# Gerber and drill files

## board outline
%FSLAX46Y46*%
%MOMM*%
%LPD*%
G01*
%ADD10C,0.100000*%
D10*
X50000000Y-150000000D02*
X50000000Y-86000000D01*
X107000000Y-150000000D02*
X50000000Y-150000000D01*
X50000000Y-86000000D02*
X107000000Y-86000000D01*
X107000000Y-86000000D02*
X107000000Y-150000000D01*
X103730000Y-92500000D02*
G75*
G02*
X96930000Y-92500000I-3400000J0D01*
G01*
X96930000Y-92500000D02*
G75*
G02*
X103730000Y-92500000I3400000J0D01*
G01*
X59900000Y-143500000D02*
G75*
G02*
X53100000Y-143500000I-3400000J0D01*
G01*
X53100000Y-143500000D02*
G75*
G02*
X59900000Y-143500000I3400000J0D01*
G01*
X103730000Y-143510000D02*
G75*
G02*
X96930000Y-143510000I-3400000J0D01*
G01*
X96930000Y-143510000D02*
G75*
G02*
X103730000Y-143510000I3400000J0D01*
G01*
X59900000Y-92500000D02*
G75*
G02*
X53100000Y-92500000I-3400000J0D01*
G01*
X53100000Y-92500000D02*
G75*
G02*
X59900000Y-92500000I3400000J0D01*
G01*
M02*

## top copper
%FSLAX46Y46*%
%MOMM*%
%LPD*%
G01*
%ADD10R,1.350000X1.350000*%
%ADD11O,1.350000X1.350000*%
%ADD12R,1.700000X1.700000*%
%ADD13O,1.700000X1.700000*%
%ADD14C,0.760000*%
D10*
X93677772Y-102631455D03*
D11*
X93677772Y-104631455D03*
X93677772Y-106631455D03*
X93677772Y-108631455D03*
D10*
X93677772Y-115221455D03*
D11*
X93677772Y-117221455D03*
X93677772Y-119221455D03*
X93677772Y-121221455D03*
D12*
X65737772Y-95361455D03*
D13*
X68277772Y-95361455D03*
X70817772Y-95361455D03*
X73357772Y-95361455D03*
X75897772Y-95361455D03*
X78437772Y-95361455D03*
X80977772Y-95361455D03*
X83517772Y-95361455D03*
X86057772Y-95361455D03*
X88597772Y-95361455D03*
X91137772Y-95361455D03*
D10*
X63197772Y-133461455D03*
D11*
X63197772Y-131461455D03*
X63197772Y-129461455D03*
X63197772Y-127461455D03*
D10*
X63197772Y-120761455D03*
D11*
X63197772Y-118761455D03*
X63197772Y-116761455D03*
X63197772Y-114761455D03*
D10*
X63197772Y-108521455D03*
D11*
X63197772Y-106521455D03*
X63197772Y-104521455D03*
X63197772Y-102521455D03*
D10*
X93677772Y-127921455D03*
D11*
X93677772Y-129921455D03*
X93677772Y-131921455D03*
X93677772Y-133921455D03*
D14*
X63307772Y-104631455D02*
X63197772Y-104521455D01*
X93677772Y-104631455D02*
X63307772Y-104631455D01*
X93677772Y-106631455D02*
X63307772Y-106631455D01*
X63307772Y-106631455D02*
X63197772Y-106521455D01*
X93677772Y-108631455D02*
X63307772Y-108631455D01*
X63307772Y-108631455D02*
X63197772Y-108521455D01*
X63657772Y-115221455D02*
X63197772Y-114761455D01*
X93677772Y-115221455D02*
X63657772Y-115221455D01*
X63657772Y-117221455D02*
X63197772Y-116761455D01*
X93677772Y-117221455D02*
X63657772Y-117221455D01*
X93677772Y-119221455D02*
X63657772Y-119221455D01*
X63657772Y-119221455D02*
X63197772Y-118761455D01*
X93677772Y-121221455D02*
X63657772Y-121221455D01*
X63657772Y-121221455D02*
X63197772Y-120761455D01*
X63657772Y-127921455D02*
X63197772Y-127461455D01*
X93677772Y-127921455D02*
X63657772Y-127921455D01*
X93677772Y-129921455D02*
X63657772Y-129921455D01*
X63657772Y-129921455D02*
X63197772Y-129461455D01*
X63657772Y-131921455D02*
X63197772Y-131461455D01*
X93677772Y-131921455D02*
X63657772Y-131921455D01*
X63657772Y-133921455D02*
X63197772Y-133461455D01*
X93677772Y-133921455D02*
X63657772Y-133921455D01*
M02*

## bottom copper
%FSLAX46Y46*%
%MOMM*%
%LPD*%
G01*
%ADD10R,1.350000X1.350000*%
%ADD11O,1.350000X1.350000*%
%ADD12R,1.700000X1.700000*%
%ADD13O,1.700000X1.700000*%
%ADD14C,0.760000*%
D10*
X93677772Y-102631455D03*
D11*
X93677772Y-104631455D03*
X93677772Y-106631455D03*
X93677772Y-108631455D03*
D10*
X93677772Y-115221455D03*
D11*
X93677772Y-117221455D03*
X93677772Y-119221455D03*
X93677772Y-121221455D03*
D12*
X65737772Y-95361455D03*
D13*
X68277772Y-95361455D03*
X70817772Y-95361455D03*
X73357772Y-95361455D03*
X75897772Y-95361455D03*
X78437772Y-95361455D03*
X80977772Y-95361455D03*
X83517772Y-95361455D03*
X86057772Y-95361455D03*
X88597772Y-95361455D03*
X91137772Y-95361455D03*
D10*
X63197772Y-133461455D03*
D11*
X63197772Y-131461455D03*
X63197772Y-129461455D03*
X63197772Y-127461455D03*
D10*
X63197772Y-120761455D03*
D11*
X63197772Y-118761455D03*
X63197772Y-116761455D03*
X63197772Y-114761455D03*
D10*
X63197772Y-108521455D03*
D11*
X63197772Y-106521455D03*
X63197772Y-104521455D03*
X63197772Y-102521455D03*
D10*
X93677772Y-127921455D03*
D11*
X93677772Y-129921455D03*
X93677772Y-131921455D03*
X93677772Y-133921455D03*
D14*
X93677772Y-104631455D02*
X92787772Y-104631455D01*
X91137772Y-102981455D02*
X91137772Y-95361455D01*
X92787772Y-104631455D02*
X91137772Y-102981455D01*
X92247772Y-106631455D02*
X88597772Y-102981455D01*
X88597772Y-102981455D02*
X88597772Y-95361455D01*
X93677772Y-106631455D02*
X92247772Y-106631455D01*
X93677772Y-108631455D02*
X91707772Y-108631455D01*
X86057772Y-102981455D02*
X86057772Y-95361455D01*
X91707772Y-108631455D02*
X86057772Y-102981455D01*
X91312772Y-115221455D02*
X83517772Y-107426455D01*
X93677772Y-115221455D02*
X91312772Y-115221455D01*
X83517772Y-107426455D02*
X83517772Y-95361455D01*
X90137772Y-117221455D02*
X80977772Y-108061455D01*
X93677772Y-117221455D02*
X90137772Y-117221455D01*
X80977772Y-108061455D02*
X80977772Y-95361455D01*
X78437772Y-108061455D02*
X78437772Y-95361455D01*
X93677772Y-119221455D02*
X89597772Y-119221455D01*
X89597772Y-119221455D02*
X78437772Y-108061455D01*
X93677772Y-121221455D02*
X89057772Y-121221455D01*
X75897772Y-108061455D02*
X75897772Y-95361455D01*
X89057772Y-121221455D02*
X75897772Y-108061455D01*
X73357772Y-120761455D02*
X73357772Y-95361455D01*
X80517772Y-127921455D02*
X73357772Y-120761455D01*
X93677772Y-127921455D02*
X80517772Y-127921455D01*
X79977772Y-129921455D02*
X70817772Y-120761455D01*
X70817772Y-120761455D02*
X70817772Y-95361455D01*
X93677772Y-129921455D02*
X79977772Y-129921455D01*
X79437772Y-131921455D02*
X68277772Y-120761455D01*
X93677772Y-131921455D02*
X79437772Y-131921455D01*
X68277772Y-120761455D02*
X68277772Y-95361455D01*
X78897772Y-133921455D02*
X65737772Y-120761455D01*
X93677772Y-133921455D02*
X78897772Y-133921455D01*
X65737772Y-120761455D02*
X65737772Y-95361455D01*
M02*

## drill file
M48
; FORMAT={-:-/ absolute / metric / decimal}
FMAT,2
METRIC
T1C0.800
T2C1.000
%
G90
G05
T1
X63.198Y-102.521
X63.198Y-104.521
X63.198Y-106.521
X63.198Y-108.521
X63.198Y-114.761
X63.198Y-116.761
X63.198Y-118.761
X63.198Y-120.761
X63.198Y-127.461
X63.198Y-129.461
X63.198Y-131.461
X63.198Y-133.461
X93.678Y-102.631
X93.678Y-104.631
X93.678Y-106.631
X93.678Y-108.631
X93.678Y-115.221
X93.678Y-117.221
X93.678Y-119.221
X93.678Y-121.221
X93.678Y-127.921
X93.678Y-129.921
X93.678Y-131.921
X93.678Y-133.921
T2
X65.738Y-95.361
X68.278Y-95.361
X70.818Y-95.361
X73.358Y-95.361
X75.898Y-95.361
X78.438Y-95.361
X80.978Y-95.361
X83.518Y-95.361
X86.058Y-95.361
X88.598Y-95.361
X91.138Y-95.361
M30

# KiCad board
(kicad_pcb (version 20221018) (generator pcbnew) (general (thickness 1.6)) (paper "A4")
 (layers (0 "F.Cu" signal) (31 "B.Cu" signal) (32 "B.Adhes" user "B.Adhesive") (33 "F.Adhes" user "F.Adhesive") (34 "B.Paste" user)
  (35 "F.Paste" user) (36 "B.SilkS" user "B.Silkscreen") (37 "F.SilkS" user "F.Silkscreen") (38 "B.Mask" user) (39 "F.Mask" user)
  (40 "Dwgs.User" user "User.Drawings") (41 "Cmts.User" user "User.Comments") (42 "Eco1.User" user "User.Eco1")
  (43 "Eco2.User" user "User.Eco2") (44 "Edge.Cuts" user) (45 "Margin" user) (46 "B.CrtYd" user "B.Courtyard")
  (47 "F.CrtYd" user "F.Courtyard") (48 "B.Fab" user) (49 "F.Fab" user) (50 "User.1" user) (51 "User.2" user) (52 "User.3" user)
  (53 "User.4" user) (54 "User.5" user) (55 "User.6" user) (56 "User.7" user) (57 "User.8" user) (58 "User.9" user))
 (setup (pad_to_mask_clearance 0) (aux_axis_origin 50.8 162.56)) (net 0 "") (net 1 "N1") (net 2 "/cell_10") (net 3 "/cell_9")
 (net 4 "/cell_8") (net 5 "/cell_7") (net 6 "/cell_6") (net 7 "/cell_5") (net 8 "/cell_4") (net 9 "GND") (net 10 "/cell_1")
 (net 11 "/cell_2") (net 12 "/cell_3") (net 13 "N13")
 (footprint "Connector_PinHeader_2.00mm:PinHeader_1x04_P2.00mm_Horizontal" (layer "F.Cu") (at 93.677772 102.631455)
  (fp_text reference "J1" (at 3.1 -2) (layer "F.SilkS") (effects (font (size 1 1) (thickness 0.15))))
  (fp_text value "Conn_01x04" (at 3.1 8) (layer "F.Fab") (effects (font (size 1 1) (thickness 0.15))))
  (pad "1" thru_hole rect (at 0 0) (size 1.35 1.35) (drill 0.8) (layers "*.Cu" "*.Mask") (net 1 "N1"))
  (pad "2" thru_hole oval (at 0 2) (size 1.35 1.35) (drill 0.8) (layers "*.Cu" "*.Mask") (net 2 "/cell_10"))
  (pad "3" thru_hole oval (at 0 4) (size 1.35 1.35) (drill 0.8) (layers "*.Cu" "*.Mask") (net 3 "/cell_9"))
  (pad "4" thru_hole oval (at 0 6) (size 1.35 1.35) (drill 0.8) (layers "*.Cu" "*.Mask") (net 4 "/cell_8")))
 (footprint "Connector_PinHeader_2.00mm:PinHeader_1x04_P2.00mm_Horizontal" (layer "F.Cu") (at 93.677772 115.221455)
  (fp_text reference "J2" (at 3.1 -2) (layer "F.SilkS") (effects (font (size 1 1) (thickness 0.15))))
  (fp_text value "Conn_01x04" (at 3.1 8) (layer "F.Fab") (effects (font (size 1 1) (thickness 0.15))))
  (pad "1" thru_hole rect (at 0 0) (size 1.35 1.35) (drill 0.8) (layers "*.Cu" "*.Mask") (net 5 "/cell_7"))
  (pad "2" thru_hole oval (at 0 2) (size 1.35 1.35) (drill 0.8) (layers "*.Cu" "*.Mask") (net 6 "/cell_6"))
  (pad "3" thru_hole oval (at 0 4) (size 1.35 1.35) (drill 0.8) (layers "*.Cu" "*.Mask") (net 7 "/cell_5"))
  (pad "4" thru_hole oval (at 0 6) (size 1.35 1.35) (drill 0.8) (layers "*.Cu" "*.Mask") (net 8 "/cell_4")))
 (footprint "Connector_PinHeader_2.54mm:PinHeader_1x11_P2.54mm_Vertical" (layer "F.Cu") (at 65.737772 95.361455 90)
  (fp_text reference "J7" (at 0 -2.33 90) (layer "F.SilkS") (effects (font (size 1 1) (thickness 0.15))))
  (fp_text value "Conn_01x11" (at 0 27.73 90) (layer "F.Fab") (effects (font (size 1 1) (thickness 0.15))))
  (pad "1" thru_hole rect (at 0 0 90) (size 1.7 1.7) (drill 1) (layers "*.Cu" "*.Mask") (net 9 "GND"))
  (pad "2" thru_hole oval (at 0 2.54 90) (size 1.7 1.7) (drill 1) (layers "*.Cu" "*.Mask") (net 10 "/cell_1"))
  (pad "3" thru_hole oval (at 0 5.08 90) (size 1.7 1.7) (drill 1) (layers "*.Cu" "*.Mask") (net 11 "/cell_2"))
  (pad "4" thru_hole oval (at 0 7.62 90) (size 1.7 1.7) (drill 1) (layers "*.Cu" "*.Mask") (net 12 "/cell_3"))
  (pad "5" thru_hole oval (at 0 10.16 90) (size 1.7 1.7) (drill 1) (layers "*.Cu" "*.Mask") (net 8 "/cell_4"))
  (pad "6" thru_hole oval (at 0 12.7 90) (size 1.7 1.7) (drill 1) (layers "*.Cu" "*.Mask") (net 7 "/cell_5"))
  (pad "7" thru_hole oval (at 0 15.24 90) (size 1.7 1.7) (drill 1) (layers "*.Cu" "*.Mask") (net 6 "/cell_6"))
  (pad "8" thru_hole oval (at 0 17.78 90) (size 1.7 1.7) (drill 1) (layers "*.Cu" "*.Mask") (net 5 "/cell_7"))
  (pad "9" thru_hole oval (at 0 20.32 90) (size 1.7 1.7) (drill 1) (layers "*.Cu" "*.Mask") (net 4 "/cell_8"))
  (pad "10" thru_hole oval (at 0 22.86 90) (size 1.7 1.7) (drill 1) (layers "*.Cu" "*.Mask") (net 3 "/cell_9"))
  (pad "11" thru_hole oval (at 0 25.4 90) (size 1.7 1.7) (drill 1) (layers "*.Cu" "*.Mask") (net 2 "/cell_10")))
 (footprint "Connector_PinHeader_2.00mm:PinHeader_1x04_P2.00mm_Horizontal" (layer "F.Cu") (at 63.197772 133.461455 180)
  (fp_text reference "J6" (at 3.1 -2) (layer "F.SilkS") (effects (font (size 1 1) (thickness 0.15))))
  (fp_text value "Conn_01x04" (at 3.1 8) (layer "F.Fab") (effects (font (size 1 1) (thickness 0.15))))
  (pad "1" thru_hole rect (at 0 0 180) (size 1.35 1.35) (drill 0.8) (layers "*.Cu" "*.Mask") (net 9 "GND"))
  (pad "2" thru_hole oval (at 0 2 180) (size 1.35 1.35) (drill 0.8) (layers "*.Cu" "*.Mask") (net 10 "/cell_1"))
  (pad "3" thru_hole oval (at 0 4 180) (size 1.35 1.35) (drill 0.8) (layers "*.Cu" "*.Mask") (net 11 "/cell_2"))
  (pad "4" thru_hole oval (at 0 6 180) (size 1.35 1.35) (drill 0.8) (layers "*.Cu" "*.Mask") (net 12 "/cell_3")))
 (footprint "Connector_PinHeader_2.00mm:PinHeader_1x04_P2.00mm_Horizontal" (layer "F.Cu") (at 63.197772 120.761455 180)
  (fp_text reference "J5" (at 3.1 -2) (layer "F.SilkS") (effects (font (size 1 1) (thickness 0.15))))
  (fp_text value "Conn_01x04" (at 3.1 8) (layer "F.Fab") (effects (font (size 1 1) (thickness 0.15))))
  (pad "1" thru_hole rect (at 0 0 180) (size 1.35 1.35) (drill 0.8) (layers "*.Cu" "*.Mask") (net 8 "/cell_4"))
  (pad "2" thru_hole oval (at 0 2 180) (size 1.35 1.35) (drill 0.8) (layers "*.Cu" "*.Mask") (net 7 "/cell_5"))
  (pad "3" thru_hole oval (at 0 4 180) (size 1.35 1.35) (drill 0.8) (layers "*.Cu" "*.Mask") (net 6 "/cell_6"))
  (pad "4" thru_hole oval (at 0 6 180) (size 1.35 1.35) (drill 0.8) (layers "*.Cu" "*.Mask") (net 5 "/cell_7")))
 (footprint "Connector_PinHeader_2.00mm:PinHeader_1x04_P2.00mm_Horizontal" (layer "F.Cu") (at 63.197772 108.521455 180)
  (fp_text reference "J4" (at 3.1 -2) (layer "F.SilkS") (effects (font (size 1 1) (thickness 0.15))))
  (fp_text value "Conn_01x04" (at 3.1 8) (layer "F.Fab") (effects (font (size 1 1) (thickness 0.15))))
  (pad "1" thru_hole rect (at 0 0 180) (size 1.35 1.35) (drill 0.8) (layers "*.Cu" "*.Mask") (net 4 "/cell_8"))
  (pad "2" thru_hole oval (at 0 2 180) (size 1.35 1.35) (drill 0.8) (layers "*.Cu" "*.Mask") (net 3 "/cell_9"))
  (pad "3" thru_hole oval (at 0 4 180) (size 1.35 1.35) (drill 0.8) (layers "*.Cu" "*.Mask") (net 2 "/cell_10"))
  (pad "4" thru_hole oval (at 0 6 180) (size 1.35 1.35) (drill 0.8) (layers "*.Cu" "*.Mask") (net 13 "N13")))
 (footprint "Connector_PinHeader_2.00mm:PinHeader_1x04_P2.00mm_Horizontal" (layer "F.Cu") (at 93.677772 127.921455)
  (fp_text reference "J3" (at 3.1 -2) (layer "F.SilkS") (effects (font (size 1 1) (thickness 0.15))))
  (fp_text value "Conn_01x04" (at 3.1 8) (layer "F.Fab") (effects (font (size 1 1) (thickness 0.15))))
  (pad "1" thru_hole rect (at 0 0) (size 1.35 1.35) (drill 0.8) (layers "*.Cu" "*.Mask") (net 12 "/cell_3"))
  (pad "2" thru_hole oval (at 0 2) (size 1.35 1.35) (drill 0.8) (layers "*.Cu" "*.Mask") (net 11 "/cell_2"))
  (pad "3" thru_hole oval (at 0 4) (size 1.35 1.35) (drill 0.8) (layers "*.Cu" "*.Mask") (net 10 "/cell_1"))
  (pad "4" thru_hole oval (at 0 6) (size 1.35 1.35) (drill 0.8) (layers "*.Cu" "*.Mask") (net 9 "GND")))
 (gr_line (start 50 150) (end 50 86) (stroke (width 0.1) (type default)) (layer "Edge.Cuts"))
 (gr_line (start 107 150) (end 50 150) (stroke (width 0.1) (type default)) (layer "Edge.Cuts"))
 (gr_line (start 50 86) (end 107 86) (stroke (width 0.1) (type default)) (layer "Edge.Cuts"))
 (gr_line (start 107 86) (end 107 150) (stroke (width 0.1) (type default)) (layer "Edge.Cuts"))
 (gr_circle (center 100.33 92.5) (end 103.73 92.5) (stroke (width 0.1) (type default)) (fill none) (layer "Edge.Cuts"))
 (gr_circle (center 56.5 143.5) (end 59.9 143.5) (stroke (width 0.1) (type default)) (fill none) (layer "Edge.Cuts"))
 (gr_circle (center 100.33 143.51) (end 103.73 143.51) (stroke (width 0.1) (type default)) (fill none) (layer "Edge.Cuts"))
 (gr_circle (center 56.5 92.5) (end 59.9 92.5) (stroke (width 0.1) (type default)) (fill none) (layer "Edge.Cuts"))
 (segment (start 63.307772 104.631455) (end 63.197772 104.521455) (width 0.76) (layer "F.Cu") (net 2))
 (segment (start 93.677772 104.631455) (end 63.307772 104.631455) (width 0.76) (layer "F.Cu") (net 2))
 (segment (start 93.677772 104.631455) (end 92.787772 104.631455) (width 0.76) (layer "B.Cu") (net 2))
 (segment (start 91.137772 102.981455) (end 91.137772 95.361455) (width 0.76) (layer "B.Cu") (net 2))
 (segment (start 92.787772 104.631455) (end 91.137772 102.981455) (width 0.76) (layer "B.Cu") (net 2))
 (segment (start 93.677772 106.631455) (end 63.307772 106.631455) (width 0.76) (layer "F.Cu") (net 3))
 (segment (start 63.307772 106.631455) (end 63.197772 106.521455) (width 0.76) (layer "F.Cu") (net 3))
 (segment (start 92.247772 106.631455) (end 88.597772 102.981455) (width 0.76) (layer "B.Cu") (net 3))
 (segment (start 88.597772 102.981455) (end 88.597772 95.361455) (width 0.76) (layer "B.Cu") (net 3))
 (segment (start 93.677772 106.631455) (end 92.247772 106.631455) (width 0.76) (layer "B.Cu") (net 3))
 (segment (start 93.677772 108.631455) (end 63.307772 108.631455) (width 0.76) (layer "F.Cu") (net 4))
 (segment (start 63.307772 108.631455) (end 63.197772 108.521455) (width 0.76) (layer "F.Cu") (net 4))
 (segment (start 93.677772 108.631455) (end 91.707772 108.631455) (width 0.76) (layer "B.Cu") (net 4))
 (segment (start 86.057772 102.981455) (end 86.057772 95.361455) (width 0.76) (layer "B.Cu") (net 4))
 (segment (start 91.707772 108.631455) (end 86.057772 102.981455) (width 0.76) (layer "B.Cu") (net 4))
 (segment (start 63.657772 115.221455) (end 63.197772 114.761455) (width 0.76) (layer "F.Cu") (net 5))
 (segment (start 93.677772 115.221455) (end 63.657772 115.221455) (width 0.76) (layer "F.Cu") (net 5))
 (segment (start 91.312772 115.221455) (end 83.517772 107.426455) (width 0.76) (layer "B.Cu") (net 5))
 (segment (start 93.677772 115.221455) (end 91.312772 115.221455) (width 0.76) (layer "B.Cu") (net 5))
 (segment (start 83.517772 107.426455) (end 83.517772 95.361455) (width 0.76) (layer "B.Cu") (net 5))
 (segment (start 63.657772 117.221455) (end 63.197772 116.761455) (width 0.76) (layer "F.Cu") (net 6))
 (segment (start 93.677772 117.221455) (end 63.657772 117.221455) (width 0.76) (layer "F.Cu") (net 6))
 (segment (start 90.137772 117.221455) (end 80.977772 108.061455) (width 0.76) (layer "B.Cu") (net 6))
 (segment (start 93.677772 117.221455) (end 90.137772 117.221455) (width 0.76) (layer "B.Cu") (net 6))
 (segment (start 80.977772 108.061455) (end 80.977772 95.361455) (width 0.76) (layer "B.Cu") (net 6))
 (segment (start 93.677772 119.221455) (end 63.657772 119.221455) (width 0.76) (layer "F.Cu") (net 7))
 (segment (start 63.657772 119.221455) (end 63.197772 118.761455) (width 0.76) (layer "F.Cu") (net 7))
 (segment (start 78.437772 108.061455) (end 78.437772 95.361455) (width 0.76) (layer "B.Cu") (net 7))
 (segment (start 93.677772 119.221455) (end 89.597772 119.221455) (width 0.76) (layer "B.Cu") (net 7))
 (segment (start 89.597772 119.221455) (end 78.437772 108.061455) (width 0.76) (layer "B.Cu") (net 7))
 (segment (start 93.677772 121.221455) (end 63.657772 121.221455) (width 0.76) (layer "F.Cu") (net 8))
 (segment (start 63.657772 121.221455) (end 63.197772 120.761455) (width 0.76) (layer "F.Cu") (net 8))
 (segment (start 93.677772 121.221455) (end 89.057772 121.221455) (width 0.76) (layer "B.Cu") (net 8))
 (segment (start 75.897772 108.061455) (end 75.897772 95.361455) (width 0.76) (layer "B.Cu") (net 8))
 (segment (start 89.057772 121.221455) (end 75.897772 108.061455) (width 0.76) (layer "B.Cu") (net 8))
 (segment (start 63.657772 127.921455) (end 63.197772 127.461455) (width 0.76) (layer "F.Cu") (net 12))
 (segment (start 93.677772 127.921455) (end 63.657772 127.921455) (width 0.76) (layer "F.Cu") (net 12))
 (segment (start 73.357772 120.761455) (end 73.357772 95.361455) (width 0.76) (layer "B.Cu") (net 12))
 (segment (start 80.517772 127.921455) (end 73.357772 120.761455) (width 0.76) (layer "B.Cu") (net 12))
 (segment (start 93.677772 127.921455) (end 80.517772 127.921455) (width 0.76) (layer "B.Cu") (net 12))
 (segment (start 93.677772 129.921455) (end 63.657772 129.921455) (width 0.76) (layer "F.Cu") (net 11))
 (segment (start 63.657772 129.921455) (end 63.197772 129.461455) (width 0.76) (layer "F.Cu") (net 11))
 (segment (start 79.977772 129.921455) (end 70.817772 120.761455) (width 0.76) (layer "B.Cu") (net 11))
 (segment (start 70.817772 120.761455) (end 70.817772 95.361455) (width 0.76) (layer "B.Cu") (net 11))
 (segment (start 93.677772 129.921455) (end 79.977772 129.921455) (width 0.76) (layer "B.Cu") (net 11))
 (segment (start 63.657772 131.921455) (end 63.197772 131.461455) (width 0.76) (layer "F.Cu") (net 10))
 (segment (start 93.677772 131.921455) (end 63.657772 131.921455) (width 0.76) (layer "F.Cu") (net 10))
 (segment (start 79.437772 131.921455) (end 68.277772 120.761455) (width 0.76) (layer "B.Cu") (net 10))
 (segment (start 93.677772 131.921455) (end 79.437772 131.921455) (width 0.76) (layer "B.Cu") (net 10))
 (segment (start 68.277772 120.761455) (end 68.277772 95.361455) (width 0.76) (layer "B.Cu") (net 10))
 (segment (start 63.657772 133.921455) (end 63.197772 133.461455) (width 0.76) (layer "F.Cu") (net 9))
 (segment (start 93.677772 133.921455) (end 63.657772 133.921455) (width 0.76) (layer "F.Cu") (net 9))
 (segment (start 78.897772 133.921455) (end 65.737772 120.761455) (width 0.76) (layer "B.Cu") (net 9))
 (segment (start 93.677772 133.921455) (end 78.897772 133.921455) (width 0.76) (layer "B.Cu") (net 9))
 (segment (start 65.737772 120.761455) (end 65.737772 95.361455) (width 0.76) (layer "B.Cu") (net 9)))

